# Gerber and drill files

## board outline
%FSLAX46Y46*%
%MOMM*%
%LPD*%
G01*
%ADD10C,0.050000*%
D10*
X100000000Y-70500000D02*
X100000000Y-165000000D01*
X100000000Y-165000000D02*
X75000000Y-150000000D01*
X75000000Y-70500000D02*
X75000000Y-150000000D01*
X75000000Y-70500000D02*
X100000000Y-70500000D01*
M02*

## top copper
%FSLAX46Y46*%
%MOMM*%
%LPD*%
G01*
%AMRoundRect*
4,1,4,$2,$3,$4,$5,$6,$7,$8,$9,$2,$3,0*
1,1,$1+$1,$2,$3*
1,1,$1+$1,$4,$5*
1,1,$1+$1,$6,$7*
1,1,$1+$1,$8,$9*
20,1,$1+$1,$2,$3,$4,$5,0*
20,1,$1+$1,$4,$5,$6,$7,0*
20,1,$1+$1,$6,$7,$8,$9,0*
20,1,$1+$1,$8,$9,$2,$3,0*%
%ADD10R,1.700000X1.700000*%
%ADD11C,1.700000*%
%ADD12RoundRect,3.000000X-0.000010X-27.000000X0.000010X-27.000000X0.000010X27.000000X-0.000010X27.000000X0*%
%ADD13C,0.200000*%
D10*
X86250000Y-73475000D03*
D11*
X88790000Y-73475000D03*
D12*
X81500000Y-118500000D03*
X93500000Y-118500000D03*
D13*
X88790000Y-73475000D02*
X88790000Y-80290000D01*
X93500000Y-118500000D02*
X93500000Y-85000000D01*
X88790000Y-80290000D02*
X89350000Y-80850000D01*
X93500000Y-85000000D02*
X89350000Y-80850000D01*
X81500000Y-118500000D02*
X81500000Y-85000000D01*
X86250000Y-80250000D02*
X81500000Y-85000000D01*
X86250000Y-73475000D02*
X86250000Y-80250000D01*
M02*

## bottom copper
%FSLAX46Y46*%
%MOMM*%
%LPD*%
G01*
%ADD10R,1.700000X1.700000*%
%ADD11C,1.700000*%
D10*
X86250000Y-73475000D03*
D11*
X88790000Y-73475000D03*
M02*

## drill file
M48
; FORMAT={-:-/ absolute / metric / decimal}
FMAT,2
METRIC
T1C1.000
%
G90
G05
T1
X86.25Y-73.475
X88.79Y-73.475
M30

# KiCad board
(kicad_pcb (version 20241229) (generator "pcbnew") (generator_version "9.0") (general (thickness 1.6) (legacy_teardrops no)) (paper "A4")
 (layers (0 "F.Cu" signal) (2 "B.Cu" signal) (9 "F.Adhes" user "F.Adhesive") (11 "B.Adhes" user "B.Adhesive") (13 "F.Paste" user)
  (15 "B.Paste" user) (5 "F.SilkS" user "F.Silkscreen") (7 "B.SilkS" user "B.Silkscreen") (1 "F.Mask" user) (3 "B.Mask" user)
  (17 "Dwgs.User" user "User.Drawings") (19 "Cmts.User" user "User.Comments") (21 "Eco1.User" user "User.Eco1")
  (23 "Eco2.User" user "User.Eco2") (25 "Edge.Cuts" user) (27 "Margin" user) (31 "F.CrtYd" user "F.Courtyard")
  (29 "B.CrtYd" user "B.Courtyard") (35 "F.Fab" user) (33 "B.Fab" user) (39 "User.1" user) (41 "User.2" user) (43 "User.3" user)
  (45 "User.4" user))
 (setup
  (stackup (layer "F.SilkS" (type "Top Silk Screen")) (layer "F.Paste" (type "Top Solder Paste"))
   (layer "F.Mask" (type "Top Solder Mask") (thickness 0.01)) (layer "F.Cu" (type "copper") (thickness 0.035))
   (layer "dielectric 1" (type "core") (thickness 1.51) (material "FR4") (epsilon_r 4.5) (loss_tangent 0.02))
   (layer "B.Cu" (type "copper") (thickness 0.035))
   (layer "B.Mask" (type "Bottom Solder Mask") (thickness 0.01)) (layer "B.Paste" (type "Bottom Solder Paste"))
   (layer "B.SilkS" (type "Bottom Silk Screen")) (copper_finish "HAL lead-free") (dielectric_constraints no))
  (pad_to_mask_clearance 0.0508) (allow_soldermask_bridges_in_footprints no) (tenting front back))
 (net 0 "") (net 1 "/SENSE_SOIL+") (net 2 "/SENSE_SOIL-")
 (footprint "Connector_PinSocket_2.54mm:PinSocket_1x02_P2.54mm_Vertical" (layer "F.Cu") (at 86.25 73.475 90)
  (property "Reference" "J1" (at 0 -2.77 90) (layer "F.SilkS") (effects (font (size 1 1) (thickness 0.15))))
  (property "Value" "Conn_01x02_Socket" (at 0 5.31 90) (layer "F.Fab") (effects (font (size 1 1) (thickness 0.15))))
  (pad "1" thru_hole rect (at 0 0 90) (size 1.7 1.7) (drill 1) (layers "*.Cu" "*.Mask") (remove_unused_layers no) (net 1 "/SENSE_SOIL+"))
  (pad "2" thru_hole circle (at 0 2.54 90) (size 1.7 1.7) (drill 1) (layers "*.Cu" "*.Mask") (remove_unused_layers no)
   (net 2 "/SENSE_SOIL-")))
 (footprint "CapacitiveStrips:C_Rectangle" (layer "F.Cu") (at 87.5 88.5)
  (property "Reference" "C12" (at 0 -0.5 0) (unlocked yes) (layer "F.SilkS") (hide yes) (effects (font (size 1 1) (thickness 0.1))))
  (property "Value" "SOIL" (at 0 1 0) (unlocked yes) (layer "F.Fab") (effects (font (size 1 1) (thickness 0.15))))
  (pad "1" smd roundrect (at -6 30) (size 6 60) (layers "F.Cu") (roundrect_rratio 0.5) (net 1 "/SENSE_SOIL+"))
  (pad "2" smd roundrect (at 6 30) (size 6 60) (layers "F.Cu") (roundrect_rratio 0.5) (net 2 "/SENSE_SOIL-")))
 (gr_line (start 100 70.5) (end 100 165) (stroke (width 0.05) (type default)) (layer "Edge.Cuts"))
 (gr_line (start 100 165) (end 75 150) (stroke (width 0.05) (type default)) (layer "Edge.Cuts"))
 (gr_line (start 75 70.5) (end 75 150) (stroke (width 0.05) (type default)) (layer "Edge.Cuts"))
 (gr_line (start 75 70.5) (end 100 70.5) (stroke (width 0.05) (type default)) (layer "Edge.Cuts"))
 (segment (start 88.79 73.475) (end 88.79 80.29) (width 0.2) (layer "F.Cu") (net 2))
 (segment (start 93.5 118.5) (end 93.5 85) (width 0.2) (layer "F.Cu") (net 2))
 (segment (start 88.79 80.29) (end 89.35 80.85) (width 0.2) (layer "F.Cu") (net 2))
 (segment (start 93.5 85) (end 89.35 80.85) (width 0.2) (layer "F.Cu") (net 2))
 (segment (start 81.5 118.5) (end 81.5 85) (width 0.2) (layer "F.Cu") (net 1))
 (segment (start 86.25 80.25) (end 81.5 85) (width 0.2) (layer "F.Cu") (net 1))
 (segment (start 86.25 73.475) (end 86.25 80.25) (width 0.2) (layer "F.Cu") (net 1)))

